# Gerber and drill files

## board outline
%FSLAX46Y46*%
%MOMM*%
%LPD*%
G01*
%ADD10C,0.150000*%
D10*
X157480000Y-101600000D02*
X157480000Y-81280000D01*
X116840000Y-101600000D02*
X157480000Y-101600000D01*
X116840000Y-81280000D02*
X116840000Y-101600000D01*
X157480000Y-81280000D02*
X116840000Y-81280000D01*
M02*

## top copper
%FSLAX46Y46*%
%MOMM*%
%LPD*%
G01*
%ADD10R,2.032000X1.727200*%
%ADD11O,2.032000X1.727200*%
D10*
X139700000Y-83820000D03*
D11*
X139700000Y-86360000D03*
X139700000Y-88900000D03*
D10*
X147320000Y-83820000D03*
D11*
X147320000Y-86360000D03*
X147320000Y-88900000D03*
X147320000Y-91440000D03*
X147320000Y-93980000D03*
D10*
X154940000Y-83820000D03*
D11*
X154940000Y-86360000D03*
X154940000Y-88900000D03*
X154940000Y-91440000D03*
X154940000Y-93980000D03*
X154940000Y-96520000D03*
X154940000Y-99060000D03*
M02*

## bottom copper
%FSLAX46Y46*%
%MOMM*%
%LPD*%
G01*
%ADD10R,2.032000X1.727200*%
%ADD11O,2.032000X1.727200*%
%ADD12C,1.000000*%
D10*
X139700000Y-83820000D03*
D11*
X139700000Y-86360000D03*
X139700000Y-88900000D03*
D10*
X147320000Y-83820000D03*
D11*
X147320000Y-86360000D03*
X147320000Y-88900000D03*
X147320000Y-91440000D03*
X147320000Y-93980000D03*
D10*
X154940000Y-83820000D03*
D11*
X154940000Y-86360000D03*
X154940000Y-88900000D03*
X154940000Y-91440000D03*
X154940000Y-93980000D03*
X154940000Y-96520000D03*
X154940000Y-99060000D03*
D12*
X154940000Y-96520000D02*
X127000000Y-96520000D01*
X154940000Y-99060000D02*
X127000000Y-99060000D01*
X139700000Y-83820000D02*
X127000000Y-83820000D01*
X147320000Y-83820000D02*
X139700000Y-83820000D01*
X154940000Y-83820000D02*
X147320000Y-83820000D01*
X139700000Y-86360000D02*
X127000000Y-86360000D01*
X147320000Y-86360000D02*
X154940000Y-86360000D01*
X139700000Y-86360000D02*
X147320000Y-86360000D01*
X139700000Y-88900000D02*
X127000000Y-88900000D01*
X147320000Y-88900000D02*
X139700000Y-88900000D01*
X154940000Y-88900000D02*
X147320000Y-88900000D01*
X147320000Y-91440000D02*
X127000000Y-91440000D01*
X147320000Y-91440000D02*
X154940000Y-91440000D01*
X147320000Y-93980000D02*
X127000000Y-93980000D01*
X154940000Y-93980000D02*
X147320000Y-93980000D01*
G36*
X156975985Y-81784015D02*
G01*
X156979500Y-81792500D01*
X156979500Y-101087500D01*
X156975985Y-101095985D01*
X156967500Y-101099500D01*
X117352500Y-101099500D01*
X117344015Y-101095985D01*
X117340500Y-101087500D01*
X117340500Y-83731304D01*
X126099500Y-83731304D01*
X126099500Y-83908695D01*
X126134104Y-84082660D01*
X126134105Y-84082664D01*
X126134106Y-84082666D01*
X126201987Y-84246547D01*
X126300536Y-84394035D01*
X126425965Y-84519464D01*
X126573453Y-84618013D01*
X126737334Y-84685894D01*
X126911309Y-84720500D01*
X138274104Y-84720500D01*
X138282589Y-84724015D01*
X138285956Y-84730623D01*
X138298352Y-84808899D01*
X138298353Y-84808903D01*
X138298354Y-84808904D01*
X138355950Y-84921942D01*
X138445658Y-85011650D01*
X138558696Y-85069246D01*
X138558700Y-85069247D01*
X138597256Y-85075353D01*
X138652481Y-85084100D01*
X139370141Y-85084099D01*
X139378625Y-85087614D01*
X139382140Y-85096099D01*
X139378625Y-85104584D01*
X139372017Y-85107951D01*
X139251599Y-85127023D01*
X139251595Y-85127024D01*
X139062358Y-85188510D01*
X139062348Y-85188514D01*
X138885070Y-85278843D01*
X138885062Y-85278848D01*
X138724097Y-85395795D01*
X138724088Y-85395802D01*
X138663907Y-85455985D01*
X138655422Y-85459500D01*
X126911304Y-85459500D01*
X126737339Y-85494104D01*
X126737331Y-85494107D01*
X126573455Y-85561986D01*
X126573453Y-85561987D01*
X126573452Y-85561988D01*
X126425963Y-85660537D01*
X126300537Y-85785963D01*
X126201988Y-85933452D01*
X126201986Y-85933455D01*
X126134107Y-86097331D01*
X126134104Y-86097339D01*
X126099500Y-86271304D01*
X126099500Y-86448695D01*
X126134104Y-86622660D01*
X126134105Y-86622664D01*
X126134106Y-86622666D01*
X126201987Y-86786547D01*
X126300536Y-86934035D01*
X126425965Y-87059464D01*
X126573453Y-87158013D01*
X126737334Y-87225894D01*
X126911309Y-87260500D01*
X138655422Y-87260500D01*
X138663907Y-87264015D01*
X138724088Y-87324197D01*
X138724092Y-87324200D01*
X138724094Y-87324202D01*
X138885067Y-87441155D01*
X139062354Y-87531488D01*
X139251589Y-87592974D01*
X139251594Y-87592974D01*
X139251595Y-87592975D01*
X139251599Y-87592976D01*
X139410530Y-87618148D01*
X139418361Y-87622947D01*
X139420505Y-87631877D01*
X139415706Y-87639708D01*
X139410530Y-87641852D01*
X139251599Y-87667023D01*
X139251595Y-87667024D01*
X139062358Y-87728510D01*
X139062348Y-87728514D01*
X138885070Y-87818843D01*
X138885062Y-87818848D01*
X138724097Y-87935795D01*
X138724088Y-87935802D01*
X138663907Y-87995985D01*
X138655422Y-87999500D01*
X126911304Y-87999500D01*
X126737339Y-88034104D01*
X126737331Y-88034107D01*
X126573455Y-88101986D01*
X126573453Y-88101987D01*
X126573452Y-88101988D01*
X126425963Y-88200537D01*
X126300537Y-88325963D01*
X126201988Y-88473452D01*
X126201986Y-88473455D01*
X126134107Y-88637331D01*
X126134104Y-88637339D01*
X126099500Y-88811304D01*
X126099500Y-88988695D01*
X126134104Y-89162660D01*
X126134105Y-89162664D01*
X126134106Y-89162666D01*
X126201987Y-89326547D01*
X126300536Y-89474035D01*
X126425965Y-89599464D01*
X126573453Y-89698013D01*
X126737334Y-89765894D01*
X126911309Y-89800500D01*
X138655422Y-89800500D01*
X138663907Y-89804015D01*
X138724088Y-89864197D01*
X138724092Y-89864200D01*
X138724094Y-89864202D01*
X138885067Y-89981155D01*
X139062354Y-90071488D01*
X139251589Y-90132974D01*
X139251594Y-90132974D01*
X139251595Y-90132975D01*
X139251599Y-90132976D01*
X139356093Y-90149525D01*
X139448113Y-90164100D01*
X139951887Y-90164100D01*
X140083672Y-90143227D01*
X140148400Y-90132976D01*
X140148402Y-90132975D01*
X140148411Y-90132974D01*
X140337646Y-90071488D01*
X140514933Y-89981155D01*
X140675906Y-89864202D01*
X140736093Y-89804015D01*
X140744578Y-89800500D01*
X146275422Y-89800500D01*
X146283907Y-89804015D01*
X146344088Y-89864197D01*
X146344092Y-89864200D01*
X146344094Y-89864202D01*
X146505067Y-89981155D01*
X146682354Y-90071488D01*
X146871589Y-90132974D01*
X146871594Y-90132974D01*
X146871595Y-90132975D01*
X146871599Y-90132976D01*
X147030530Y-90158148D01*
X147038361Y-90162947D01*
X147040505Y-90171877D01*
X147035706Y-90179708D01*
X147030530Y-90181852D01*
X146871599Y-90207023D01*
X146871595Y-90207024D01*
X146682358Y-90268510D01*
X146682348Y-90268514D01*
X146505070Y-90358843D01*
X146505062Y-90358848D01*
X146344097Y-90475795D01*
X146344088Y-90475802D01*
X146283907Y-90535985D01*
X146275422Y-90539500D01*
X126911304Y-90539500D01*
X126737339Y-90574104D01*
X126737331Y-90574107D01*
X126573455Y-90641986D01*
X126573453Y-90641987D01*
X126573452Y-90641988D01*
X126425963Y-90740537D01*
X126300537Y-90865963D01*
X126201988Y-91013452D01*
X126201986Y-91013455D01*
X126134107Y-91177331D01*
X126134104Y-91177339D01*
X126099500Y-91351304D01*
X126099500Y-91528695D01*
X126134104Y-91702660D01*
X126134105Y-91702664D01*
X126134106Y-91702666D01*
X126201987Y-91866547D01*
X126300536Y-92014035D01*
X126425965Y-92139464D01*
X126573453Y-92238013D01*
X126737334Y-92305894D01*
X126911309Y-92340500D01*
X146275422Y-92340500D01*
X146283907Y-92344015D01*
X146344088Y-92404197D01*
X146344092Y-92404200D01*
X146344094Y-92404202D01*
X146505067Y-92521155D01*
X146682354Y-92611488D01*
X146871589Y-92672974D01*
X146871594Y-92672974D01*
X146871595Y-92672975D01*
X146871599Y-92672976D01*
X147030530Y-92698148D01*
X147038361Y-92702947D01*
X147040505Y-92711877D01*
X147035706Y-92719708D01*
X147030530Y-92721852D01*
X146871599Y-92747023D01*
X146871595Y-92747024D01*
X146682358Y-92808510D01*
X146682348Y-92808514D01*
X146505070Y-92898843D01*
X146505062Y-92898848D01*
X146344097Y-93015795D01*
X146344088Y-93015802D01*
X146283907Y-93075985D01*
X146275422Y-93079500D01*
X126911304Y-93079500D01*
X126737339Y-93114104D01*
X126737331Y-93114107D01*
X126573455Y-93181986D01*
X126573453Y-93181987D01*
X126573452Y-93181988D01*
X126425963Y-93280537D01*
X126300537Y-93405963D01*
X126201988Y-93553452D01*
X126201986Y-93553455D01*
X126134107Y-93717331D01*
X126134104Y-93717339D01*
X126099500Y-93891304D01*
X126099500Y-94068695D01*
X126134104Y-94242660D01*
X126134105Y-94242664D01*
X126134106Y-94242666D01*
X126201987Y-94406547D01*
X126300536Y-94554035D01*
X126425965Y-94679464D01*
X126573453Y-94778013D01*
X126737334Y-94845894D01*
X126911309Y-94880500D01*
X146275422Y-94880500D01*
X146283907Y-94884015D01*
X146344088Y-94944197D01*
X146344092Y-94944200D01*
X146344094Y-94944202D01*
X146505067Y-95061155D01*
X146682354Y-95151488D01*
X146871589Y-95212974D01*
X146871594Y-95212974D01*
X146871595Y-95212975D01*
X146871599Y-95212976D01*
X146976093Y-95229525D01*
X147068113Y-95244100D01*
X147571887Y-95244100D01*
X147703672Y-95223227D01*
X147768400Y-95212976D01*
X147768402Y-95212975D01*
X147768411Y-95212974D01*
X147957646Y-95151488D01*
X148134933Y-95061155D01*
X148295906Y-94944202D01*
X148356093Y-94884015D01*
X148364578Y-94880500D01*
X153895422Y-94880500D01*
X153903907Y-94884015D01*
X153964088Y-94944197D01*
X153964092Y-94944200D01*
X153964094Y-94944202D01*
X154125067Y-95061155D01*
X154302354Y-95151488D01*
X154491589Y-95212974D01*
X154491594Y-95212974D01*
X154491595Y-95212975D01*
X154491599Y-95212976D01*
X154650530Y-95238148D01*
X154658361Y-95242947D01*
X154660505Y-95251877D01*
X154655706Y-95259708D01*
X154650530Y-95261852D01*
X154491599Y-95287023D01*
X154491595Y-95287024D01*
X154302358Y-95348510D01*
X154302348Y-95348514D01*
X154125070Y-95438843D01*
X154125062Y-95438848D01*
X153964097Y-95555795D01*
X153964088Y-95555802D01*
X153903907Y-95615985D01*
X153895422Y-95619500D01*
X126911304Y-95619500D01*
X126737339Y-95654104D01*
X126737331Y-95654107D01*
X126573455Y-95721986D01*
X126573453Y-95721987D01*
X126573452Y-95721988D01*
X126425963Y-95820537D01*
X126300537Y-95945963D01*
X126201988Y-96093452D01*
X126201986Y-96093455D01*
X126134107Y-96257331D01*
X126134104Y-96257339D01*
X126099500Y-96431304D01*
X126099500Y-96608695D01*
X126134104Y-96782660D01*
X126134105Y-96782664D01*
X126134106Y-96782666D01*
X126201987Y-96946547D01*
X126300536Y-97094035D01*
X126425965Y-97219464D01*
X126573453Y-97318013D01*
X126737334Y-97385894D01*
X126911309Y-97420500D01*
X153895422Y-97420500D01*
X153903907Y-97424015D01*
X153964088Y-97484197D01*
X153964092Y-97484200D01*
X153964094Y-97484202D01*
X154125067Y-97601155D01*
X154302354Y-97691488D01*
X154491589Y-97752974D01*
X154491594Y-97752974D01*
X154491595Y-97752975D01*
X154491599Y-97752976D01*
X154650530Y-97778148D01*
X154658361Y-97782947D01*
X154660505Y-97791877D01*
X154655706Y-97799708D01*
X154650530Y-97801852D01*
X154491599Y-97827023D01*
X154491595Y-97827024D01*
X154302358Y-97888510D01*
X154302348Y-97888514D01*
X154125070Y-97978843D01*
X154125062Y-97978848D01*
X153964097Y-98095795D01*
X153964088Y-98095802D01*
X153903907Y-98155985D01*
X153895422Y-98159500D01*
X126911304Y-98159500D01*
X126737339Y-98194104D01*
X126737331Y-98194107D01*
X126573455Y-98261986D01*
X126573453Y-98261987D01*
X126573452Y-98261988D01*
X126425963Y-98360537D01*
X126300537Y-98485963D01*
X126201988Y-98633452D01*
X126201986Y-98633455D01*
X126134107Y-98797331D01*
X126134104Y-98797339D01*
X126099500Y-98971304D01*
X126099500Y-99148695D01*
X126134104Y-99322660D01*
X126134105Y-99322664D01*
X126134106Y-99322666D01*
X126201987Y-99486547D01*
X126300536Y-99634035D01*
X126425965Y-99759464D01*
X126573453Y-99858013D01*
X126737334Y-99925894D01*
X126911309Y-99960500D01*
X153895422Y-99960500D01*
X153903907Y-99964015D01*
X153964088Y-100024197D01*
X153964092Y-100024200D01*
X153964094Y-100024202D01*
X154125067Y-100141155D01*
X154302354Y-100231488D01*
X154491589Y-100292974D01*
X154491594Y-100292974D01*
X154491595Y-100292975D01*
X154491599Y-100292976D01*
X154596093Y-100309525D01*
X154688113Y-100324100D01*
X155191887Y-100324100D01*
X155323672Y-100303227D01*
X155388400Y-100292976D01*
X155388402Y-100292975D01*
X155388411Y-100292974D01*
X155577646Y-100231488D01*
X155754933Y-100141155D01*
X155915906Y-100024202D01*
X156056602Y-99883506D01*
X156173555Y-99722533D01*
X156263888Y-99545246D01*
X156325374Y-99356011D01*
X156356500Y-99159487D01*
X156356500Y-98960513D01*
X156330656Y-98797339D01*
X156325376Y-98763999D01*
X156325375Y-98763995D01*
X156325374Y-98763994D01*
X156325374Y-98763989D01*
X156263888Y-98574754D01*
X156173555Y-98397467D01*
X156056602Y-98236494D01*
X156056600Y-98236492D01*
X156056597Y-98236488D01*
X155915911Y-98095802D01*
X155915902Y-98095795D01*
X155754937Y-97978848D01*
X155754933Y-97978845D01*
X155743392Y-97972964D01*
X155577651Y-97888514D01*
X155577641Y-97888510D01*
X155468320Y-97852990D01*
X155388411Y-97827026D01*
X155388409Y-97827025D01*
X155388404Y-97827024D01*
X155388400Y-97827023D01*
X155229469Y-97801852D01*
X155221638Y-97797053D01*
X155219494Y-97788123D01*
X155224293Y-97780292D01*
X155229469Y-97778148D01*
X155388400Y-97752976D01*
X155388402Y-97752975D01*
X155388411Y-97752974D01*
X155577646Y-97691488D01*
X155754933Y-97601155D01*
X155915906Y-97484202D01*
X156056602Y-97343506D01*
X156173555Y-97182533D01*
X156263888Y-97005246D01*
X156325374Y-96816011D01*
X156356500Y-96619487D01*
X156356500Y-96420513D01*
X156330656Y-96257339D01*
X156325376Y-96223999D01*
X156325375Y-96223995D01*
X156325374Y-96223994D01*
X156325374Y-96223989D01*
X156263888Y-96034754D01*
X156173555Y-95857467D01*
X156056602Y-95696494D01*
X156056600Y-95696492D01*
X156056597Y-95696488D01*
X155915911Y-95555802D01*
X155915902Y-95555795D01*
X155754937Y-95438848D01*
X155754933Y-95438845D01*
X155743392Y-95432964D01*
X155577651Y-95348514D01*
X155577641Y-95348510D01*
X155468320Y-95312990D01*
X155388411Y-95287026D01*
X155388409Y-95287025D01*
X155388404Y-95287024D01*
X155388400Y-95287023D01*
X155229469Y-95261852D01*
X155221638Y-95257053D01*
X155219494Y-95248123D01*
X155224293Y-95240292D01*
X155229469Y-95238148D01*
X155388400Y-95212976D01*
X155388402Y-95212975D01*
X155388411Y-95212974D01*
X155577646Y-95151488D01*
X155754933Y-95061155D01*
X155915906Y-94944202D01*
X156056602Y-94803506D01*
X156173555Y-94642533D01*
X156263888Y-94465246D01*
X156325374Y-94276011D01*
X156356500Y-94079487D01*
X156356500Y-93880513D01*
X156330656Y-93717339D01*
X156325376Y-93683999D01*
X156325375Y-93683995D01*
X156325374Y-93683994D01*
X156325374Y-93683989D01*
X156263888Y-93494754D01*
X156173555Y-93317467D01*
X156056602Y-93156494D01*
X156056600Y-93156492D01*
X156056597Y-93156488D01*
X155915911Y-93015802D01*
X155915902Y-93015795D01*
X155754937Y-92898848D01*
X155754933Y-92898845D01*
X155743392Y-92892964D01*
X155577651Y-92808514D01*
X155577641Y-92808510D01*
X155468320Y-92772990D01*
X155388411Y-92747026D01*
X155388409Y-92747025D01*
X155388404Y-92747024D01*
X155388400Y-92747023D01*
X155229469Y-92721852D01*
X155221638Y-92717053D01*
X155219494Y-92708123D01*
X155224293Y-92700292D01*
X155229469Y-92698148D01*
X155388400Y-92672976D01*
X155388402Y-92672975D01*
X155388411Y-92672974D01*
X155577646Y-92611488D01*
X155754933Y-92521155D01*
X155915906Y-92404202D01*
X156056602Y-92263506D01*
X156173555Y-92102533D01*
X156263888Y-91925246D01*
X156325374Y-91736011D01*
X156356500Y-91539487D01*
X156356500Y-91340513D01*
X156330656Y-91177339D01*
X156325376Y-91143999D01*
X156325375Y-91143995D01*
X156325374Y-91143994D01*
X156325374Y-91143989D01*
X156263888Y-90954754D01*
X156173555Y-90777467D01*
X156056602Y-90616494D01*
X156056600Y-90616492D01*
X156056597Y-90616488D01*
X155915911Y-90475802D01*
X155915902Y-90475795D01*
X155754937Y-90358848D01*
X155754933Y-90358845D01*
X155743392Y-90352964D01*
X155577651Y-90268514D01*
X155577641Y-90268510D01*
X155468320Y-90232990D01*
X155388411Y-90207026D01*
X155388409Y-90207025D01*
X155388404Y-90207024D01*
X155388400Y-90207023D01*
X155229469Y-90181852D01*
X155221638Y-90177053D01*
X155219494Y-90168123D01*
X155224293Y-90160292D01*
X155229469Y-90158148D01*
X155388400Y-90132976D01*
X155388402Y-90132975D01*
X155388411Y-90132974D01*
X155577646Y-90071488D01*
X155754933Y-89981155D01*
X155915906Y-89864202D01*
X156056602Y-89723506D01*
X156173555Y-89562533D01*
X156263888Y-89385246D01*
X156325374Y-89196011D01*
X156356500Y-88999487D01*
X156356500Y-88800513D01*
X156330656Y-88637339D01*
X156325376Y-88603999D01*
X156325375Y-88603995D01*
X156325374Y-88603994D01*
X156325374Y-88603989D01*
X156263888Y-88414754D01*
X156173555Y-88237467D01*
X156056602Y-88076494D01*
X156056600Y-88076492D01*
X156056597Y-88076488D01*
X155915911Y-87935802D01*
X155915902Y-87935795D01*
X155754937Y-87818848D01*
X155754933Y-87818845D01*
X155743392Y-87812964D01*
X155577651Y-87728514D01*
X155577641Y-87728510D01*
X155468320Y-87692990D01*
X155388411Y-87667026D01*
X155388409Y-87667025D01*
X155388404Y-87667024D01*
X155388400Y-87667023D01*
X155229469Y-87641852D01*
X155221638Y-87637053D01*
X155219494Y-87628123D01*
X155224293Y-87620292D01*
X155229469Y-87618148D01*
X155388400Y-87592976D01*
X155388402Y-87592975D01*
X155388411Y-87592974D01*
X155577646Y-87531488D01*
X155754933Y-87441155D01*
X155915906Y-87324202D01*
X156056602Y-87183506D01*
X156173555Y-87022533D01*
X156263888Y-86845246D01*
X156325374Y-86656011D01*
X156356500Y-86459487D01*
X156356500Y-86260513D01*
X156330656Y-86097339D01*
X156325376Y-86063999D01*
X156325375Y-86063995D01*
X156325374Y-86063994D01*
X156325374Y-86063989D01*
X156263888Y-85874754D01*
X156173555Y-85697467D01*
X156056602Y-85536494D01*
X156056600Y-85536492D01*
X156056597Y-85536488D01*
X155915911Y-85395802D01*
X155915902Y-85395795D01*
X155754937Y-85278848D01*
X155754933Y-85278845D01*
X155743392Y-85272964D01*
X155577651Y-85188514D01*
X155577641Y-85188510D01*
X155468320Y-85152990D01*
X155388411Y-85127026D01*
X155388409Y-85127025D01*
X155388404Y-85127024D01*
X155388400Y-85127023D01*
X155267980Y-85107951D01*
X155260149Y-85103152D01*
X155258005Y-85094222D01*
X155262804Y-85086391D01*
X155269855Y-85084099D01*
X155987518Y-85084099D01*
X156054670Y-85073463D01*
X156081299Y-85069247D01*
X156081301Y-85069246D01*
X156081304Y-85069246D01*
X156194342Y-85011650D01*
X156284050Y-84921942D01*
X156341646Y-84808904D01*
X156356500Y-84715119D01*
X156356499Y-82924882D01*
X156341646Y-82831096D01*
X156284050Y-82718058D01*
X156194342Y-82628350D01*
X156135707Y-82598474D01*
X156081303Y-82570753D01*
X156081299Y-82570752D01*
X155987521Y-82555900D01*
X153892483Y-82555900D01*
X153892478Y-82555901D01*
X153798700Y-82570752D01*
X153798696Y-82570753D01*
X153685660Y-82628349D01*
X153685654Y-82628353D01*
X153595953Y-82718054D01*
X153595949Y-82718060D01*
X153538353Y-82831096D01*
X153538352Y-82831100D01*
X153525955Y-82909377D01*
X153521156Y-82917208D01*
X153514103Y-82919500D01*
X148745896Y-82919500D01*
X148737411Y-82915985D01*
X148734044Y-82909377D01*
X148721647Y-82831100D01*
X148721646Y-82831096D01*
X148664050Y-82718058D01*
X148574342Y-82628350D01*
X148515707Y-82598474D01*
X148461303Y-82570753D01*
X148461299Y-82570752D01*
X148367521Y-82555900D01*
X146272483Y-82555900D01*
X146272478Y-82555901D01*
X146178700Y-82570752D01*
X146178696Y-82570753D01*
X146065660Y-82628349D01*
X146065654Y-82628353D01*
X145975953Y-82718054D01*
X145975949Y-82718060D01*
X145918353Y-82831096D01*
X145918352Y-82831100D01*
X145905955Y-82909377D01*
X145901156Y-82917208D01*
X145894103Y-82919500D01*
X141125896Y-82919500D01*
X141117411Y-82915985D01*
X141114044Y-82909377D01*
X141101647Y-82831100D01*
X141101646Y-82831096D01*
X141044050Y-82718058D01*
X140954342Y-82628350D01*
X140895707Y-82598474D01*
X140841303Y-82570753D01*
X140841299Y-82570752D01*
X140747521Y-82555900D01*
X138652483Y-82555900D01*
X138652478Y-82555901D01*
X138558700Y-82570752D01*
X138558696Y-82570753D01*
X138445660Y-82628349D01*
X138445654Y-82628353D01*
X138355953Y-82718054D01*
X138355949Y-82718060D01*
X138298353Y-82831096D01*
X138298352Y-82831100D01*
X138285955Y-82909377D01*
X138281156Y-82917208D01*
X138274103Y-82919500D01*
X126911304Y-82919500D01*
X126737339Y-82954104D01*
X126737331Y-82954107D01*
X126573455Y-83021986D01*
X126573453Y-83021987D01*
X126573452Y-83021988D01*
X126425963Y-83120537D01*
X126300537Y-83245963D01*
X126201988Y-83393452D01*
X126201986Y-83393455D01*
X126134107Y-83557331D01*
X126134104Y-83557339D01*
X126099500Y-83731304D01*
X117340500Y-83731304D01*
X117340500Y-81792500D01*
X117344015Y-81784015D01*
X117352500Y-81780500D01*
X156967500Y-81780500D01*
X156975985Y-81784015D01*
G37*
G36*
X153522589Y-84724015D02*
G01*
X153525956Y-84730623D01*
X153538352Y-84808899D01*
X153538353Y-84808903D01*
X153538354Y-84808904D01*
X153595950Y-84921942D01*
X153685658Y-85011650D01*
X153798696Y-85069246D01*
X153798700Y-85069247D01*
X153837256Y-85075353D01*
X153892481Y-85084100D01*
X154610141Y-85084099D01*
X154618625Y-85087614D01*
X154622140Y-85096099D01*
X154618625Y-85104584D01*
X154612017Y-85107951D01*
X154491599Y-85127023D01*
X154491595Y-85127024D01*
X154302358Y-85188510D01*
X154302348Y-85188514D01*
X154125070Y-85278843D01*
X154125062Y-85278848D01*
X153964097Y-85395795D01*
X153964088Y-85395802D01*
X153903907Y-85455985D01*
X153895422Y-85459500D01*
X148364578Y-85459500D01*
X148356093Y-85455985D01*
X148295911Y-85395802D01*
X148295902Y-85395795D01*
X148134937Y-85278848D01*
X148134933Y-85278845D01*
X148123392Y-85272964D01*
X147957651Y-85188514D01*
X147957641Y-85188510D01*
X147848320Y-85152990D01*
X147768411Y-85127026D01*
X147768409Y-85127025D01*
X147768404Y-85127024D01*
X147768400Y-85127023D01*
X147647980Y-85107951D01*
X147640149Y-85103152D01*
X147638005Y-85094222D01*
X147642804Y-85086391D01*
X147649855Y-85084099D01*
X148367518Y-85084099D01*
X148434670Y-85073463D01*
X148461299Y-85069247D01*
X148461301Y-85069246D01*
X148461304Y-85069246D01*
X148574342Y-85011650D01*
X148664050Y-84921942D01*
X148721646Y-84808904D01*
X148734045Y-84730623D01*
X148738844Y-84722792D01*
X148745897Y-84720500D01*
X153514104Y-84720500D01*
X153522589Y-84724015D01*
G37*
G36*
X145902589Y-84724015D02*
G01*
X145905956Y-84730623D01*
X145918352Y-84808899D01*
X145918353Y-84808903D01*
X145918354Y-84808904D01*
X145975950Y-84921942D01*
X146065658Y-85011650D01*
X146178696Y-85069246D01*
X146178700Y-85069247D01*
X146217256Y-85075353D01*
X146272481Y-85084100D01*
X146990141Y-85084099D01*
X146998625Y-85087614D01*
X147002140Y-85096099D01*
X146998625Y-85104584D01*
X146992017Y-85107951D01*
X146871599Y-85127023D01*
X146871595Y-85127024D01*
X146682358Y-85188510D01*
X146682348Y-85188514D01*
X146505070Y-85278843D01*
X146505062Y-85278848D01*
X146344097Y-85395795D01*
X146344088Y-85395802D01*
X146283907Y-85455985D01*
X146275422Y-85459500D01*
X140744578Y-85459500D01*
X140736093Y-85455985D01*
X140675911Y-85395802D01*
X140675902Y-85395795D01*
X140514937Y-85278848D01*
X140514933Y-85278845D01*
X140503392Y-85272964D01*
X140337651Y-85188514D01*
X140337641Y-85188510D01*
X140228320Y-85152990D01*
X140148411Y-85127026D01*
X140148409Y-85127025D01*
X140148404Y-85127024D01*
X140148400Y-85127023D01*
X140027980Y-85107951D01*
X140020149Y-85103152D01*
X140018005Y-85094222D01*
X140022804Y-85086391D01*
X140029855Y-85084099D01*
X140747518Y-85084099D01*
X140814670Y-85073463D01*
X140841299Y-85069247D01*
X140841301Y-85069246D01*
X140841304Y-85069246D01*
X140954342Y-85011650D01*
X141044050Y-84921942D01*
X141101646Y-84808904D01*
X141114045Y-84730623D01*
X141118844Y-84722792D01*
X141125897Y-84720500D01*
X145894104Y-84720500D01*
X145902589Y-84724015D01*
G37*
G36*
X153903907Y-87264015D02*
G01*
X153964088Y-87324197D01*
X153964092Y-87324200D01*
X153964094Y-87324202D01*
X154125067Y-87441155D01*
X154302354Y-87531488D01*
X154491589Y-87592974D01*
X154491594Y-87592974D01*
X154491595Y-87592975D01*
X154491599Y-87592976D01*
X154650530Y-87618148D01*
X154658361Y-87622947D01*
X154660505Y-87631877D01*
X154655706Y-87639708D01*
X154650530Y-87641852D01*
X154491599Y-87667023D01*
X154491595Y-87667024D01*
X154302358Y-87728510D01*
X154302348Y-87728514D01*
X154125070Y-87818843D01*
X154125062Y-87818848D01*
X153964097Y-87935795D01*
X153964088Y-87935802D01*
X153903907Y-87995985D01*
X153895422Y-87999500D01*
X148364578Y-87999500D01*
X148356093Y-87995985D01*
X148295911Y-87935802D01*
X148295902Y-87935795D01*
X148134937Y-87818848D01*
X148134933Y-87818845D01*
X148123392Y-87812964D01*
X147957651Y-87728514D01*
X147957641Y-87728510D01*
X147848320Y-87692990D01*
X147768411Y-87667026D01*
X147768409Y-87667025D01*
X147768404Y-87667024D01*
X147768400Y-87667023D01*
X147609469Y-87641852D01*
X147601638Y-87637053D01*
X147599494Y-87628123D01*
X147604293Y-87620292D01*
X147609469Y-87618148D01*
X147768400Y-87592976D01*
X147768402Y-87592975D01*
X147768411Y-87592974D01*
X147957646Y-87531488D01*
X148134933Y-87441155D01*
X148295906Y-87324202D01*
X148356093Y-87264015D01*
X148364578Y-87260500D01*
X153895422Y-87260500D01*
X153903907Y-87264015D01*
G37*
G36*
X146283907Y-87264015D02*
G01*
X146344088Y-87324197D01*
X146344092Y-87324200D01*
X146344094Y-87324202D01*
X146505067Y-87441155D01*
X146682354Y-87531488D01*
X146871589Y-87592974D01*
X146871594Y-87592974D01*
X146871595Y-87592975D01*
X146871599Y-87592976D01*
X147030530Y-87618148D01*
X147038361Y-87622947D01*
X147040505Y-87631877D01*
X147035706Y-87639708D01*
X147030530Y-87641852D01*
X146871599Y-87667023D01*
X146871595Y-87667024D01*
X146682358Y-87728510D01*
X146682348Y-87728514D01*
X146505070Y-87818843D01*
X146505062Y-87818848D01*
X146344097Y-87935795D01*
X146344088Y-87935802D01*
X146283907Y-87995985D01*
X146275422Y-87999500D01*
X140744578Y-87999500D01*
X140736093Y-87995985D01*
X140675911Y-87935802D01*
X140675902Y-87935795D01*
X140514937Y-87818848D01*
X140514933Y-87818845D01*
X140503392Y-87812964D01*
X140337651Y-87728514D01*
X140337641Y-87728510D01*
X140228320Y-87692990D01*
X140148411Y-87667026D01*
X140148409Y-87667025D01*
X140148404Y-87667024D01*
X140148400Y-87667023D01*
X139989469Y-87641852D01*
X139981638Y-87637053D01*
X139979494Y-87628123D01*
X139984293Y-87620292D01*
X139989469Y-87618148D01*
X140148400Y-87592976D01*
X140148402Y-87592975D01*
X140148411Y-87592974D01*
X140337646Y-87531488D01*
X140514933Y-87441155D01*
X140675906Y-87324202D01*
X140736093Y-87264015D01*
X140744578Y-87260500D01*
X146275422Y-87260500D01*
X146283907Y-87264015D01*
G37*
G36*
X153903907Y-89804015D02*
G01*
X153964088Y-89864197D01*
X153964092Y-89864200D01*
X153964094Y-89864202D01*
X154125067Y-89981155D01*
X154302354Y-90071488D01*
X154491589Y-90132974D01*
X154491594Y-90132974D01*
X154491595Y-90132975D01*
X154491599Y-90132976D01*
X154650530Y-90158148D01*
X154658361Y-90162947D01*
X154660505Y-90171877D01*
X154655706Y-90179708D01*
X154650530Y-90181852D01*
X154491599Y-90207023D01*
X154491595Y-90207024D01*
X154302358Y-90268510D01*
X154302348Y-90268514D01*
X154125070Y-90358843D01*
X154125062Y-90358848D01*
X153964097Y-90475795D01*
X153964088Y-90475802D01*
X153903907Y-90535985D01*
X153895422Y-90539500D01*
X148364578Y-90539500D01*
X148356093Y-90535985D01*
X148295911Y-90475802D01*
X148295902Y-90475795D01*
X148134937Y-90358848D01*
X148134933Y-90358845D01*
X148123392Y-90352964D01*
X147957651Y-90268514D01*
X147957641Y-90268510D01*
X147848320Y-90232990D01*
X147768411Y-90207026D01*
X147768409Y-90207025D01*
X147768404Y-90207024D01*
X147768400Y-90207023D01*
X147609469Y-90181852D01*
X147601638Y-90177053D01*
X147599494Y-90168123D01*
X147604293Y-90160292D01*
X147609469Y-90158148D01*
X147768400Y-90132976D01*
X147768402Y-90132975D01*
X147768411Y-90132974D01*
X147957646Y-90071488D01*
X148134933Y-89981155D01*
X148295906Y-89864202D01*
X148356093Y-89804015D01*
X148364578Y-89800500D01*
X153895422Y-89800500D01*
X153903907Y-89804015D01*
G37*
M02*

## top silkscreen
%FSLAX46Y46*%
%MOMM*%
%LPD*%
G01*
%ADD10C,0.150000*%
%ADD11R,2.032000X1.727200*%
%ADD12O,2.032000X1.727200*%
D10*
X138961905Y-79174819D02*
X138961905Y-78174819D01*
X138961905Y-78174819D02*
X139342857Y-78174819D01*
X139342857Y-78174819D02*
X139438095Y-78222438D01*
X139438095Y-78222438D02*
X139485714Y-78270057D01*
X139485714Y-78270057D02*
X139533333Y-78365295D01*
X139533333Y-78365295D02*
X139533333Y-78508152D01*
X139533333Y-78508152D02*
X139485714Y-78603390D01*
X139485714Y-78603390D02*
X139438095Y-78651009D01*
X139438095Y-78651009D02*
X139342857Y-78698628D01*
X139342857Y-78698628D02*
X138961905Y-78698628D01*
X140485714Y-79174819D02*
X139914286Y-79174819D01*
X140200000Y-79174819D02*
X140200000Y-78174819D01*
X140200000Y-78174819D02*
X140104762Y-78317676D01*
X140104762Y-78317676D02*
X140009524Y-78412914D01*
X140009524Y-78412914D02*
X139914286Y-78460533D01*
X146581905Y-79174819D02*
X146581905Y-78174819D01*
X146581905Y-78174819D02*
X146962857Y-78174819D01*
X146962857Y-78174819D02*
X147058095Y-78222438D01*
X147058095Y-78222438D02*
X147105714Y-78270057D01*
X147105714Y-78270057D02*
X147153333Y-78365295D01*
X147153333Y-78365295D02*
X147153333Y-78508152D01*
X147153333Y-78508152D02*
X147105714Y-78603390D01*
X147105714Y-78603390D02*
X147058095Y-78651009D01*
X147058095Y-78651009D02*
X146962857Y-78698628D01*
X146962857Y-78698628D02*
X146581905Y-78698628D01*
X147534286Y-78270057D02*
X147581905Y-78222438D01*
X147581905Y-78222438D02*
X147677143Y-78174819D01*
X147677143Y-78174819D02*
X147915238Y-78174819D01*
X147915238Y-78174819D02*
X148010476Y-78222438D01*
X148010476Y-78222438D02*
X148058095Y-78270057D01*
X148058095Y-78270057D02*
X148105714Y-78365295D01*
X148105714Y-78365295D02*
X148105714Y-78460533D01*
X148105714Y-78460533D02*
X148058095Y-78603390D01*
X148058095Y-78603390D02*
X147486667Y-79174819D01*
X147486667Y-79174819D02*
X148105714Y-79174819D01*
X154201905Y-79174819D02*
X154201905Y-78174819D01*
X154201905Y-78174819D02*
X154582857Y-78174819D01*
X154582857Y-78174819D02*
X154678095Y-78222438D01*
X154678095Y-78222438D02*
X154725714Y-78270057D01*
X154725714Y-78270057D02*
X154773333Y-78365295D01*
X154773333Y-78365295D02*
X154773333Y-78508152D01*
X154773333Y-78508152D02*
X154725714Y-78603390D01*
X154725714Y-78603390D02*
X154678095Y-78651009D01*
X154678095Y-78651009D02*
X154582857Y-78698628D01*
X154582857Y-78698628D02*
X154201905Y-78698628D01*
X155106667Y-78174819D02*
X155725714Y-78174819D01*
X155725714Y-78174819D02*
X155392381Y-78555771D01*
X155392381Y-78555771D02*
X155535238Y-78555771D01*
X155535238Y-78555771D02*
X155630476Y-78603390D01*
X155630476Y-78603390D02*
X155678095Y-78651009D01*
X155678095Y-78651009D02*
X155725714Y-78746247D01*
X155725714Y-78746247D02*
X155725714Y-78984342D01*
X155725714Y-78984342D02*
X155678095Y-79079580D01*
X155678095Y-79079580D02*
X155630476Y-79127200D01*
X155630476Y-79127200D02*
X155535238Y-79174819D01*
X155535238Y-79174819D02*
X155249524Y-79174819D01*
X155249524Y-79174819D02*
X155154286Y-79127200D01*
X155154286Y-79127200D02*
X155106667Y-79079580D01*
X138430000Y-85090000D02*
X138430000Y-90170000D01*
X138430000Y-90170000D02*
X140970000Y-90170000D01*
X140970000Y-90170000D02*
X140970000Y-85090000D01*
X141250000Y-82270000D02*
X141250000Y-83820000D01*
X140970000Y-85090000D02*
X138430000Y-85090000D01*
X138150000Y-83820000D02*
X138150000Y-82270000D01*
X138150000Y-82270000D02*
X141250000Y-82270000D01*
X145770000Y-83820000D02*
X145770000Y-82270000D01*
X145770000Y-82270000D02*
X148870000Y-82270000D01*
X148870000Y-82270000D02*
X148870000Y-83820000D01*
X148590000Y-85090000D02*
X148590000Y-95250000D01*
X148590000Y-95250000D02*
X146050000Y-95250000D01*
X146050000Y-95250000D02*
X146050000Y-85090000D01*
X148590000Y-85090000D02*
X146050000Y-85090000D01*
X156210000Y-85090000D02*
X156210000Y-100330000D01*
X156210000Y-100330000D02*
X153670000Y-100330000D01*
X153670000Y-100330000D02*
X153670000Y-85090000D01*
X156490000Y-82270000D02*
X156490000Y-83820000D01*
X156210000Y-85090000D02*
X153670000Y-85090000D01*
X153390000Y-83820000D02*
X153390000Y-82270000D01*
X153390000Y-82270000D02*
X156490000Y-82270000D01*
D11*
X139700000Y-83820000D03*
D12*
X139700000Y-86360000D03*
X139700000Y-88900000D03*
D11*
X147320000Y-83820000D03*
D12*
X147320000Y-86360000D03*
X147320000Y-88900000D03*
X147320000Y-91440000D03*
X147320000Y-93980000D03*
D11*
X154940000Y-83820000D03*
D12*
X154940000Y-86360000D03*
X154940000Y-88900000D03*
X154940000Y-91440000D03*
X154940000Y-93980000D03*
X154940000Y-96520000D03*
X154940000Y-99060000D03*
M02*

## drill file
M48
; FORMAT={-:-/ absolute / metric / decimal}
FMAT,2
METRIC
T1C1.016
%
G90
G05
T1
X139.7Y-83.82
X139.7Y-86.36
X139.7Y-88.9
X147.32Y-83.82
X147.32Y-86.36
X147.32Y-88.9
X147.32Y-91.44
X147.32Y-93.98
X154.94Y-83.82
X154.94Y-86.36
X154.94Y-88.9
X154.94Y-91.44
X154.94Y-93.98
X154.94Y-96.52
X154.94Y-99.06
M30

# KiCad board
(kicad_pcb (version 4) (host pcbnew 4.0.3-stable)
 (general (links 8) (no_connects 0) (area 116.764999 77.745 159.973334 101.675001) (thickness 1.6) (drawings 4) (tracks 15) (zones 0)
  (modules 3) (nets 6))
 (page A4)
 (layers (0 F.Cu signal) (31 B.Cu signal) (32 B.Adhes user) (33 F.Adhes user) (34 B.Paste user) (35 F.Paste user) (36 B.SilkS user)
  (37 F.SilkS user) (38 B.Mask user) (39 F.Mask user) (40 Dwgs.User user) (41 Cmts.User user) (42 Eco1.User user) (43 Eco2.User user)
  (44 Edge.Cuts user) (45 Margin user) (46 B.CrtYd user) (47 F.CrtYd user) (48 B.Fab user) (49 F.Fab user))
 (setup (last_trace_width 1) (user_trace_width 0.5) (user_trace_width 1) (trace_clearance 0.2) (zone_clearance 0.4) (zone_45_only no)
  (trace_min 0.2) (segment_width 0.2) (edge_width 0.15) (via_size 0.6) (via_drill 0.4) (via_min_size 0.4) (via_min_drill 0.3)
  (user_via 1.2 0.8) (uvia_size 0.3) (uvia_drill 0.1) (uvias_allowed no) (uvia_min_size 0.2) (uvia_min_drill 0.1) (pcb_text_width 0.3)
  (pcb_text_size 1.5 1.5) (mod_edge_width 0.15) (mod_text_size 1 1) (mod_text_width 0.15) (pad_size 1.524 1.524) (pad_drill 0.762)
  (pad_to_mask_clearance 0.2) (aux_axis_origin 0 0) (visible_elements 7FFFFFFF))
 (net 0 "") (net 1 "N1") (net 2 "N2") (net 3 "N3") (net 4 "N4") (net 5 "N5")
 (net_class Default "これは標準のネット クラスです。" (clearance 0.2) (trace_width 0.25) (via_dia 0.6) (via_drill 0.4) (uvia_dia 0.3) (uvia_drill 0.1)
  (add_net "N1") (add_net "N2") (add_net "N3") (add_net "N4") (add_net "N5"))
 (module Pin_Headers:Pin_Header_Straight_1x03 (layer F.Cu) (at 139.7 83.82)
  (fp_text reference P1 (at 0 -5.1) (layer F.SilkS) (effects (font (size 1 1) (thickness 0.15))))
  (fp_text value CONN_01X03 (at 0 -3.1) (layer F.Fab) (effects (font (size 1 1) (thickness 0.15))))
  (fp_line (start -1.27 1.27) (end -1.27 6.35) (layer F.SilkS) (width 0.15))
  (fp_line (start -1.27 6.35) (end 1.27 6.35) (layer F.SilkS) (width 0.15))
  (fp_line (start 1.27 6.35) (end 1.27 1.27) (layer F.SilkS) (width 0.15))
  (fp_line (start 1.55 -1.55) (end 1.55 0) (layer F.SilkS) (width 0.15))
  (fp_line (start 1.27 1.27) (end -1.27 1.27) (layer F.SilkS) (width 0.15))
  (fp_line (start -1.55 0) (end -1.55 -1.55) (layer F.SilkS) (width 0.15))
  (fp_line (start -1.55 -1.55) (end 1.55 -1.55) (layer F.SilkS) (width 0.15))
  (pad 1 thru_hole rect (at 0 0) (size 2.032 1.7272) (drill 1.016) (layers *.Cu *.Mask F.SilkS) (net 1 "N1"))
  (pad 2 thru_hole oval (at 0 2.54) (size 2.032 1.7272) (drill 1.016) (layers *.Cu *.Mask F.SilkS) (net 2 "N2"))
  (pad 3 thru_hole oval (at 0 5.08) (size 2.032 1.7272) (drill 1.016) (layers *.Cu *.Mask F.SilkS) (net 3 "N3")))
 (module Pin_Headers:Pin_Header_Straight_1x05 (layer F.Cu) (at 147.32 83.82)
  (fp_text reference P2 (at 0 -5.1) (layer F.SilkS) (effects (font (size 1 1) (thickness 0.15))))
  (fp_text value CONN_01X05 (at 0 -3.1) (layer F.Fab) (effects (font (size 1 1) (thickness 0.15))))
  (fp_line (start -1.55 0) (end -1.55 -1.55) (layer F.SilkS) (width 0.15))
  (fp_line (start -1.55 -1.55) (end 1.55 -1.55) (layer F.SilkS) (width 0.15))
  (fp_line (start 1.55 -1.55) (end 1.55 0) (layer F.SilkS) (width 0.15))
  (fp_line (start 1.27 1.27) (end 1.27 11.43) (layer F.SilkS) (width 0.15))
  (fp_line (start 1.27 11.43) (end -1.27 11.43) (layer F.SilkS) (width 0.15))
  (fp_line (start -1.27 11.43) (end -1.27 1.27) (layer F.SilkS) (width 0.15))
  (fp_line (start 1.27 1.27) (end -1.27 1.27) (layer F.SilkS) (width 0.15))
  (pad 1 thru_hole rect (at 0 0) (size 2.032 1.7272) (drill 1.016) (layers *.Cu *.Mask F.SilkS) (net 1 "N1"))
  (pad 2 thru_hole oval (at 0 2.54) (size 2.032 1.7272) (drill 1.016) (layers *.Cu *.Mask F.SilkS) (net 2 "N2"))
  (pad 3 thru_hole oval (at 0 5.08) (size 2.032 1.7272) (drill 1.016) (layers *.Cu *.Mask F.SilkS) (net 3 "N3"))
  (pad 4 thru_hole oval (at 0 7.62) (size 2.032 1.7272) (drill 1.016) (layers *.Cu *.Mask F.SilkS) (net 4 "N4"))
  (pad 5 thru_hole oval (at 0 10.16) (size 2.032 1.7272) (drill 1.016) (layers *.Cu *.Mask F.SilkS) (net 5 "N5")))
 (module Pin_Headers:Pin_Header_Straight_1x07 (layer F.Cu) (at 154.94 83.82)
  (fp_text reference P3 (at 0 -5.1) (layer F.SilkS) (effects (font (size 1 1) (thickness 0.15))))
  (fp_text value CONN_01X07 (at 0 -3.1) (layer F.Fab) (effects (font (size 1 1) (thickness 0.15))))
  (fp_line (start 1.27 1.27) (end 1.27 16.51) (layer F.SilkS) (width 0.15))
  (fp_line (start 1.27 16.51) (end -1.27 16.51) (layer F.SilkS) (width 0.15))
  (fp_line (start -1.27 16.51) (end -1.27 1.27) (layer F.SilkS) (width 0.15))
  (fp_line (start 1.55 -1.55) (end 1.55 0) (layer F.SilkS) (width 0.15))
  (fp_line (start 1.27 1.27) (end -1.27 1.27) (layer F.SilkS) (width 0.15))
  (fp_line (start -1.55 0) (end -1.55 -1.55) (layer F.SilkS) (width 0.15))
  (fp_line (start -1.55 -1.55) (end 1.55 -1.55) (layer F.SilkS) (width 0.15))
  (pad 1 thru_hole rect (at 0 0) (size 2.032 1.7272) (drill 1.016) (layers *.Cu *.Mask F.SilkS) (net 1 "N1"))
  (pad 2 thru_hole oval (at 0 2.54) (size 2.032 1.7272) (drill 1.016) (layers *.Cu *.Mask F.SilkS) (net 2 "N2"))
  (pad 3 thru_hole oval (at 0 5.08) (size 2.032 1.7272) (drill 1.016) (layers *.Cu *.Mask F.SilkS) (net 3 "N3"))
  (pad 4 thru_hole oval (at 0 7.62) (size 2.032 1.7272) (drill 1.016) (layers *.Cu *.Mask F.SilkS) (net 4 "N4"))
  (pad 5 thru_hole oval (at 0 10.16) (size 2.032 1.7272) (drill 1.016) (layers *.Cu *.Mask F.SilkS) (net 5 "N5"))
  (pad 6 thru_hole oval (at 0 12.7) (size 2.032 1.7272) (drill 1.016) (layers *.Cu *.Mask F.SilkS))
  (pad 7 thru_hole oval (at 0 15.24) (size 2.032 1.7272) (drill 1.016) (layers *.Cu *.Mask F.SilkS)))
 (gr_line (start 157.48 101.6) (end 157.48 81.28) (angle 90) (layer Edge.Cuts) (width 0.15))
 (gr_line (start 116.84 101.6) (end 157.48 101.6) (angle 90) (layer Edge.Cuts) (width 0.15))
 (gr_line (start 116.84 81.28) (end 116.84 101.6) (angle 90) (layer Edge.Cuts) (width 0.15))
 (gr_line (start 157.48 81.28) (end 116.84 81.28) (angle 90) (layer Edge.Cuts) (width 0.15))
 (segment (start 154.94 96.52) (end 127 96.52) (width 1) (layer B.Cu) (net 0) (status 400000))
 (segment (start 154.94 99.06) (end 127 99.06) (width 1) (layer B.Cu) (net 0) (status 400000))
 (segment (start 139.7 83.82) (end 127 83.82) (width 1) (layer B.Cu) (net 1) (status 400000))
 (segment (start 147.32 83.82) (end 139.7 83.82) (width 1) (layer B.Cu) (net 1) (status C00000))
 (segment (start 154.94 83.82) (end 147.32 83.82) (width 1) (layer B.Cu) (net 1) (status C00000))
 (segment (start 139.7 86.36) (end 127 86.36) (width 1) (layer B.Cu) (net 2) (status 400000))
 (segment (start 147.32 86.36) (end 154.94 86.36) (width 1) (layer B.Cu) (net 2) (status C00000))
 (segment (start 139.7 86.36) (end 147.32 86.36) (width 1) (layer B.Cu) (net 2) (status C00000))
 (segment (start 139.7 88.9) (end 127 88.9) (width 1) (layer B.Cu) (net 3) (status 400000))
 (segment (start 147.32 88.9) (end 139.7 88.9) (width 1) (layer B.Cu) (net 3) (status C00000))
 (segment (start 154.94 88.9) (end 147.32 88.9) (width 1) (layer B.Cu) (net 3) (status C00000))
 (segment (start 147.32 91.44) (end 127 91.44) (width 1) (layer B.Cu) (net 4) (status 400000))
 (segment (start 147.32 91.44) (end 154.94 91.44) (width 1) (layer B.Cu) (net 4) (status C00000))
 (segment (start 147.32 93.98) (end 127 93.98) (width 1) (layer B.Cu) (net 5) (status 400000))
 (segment (start 154.94 93.98) (end 147.32 93.98) (width 1) (layer B.Cu) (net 5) (status C00000))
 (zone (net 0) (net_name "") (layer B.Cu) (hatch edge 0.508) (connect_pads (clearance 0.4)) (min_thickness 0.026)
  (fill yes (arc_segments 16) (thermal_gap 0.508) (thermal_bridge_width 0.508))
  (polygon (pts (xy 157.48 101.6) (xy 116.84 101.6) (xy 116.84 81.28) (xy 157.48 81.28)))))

